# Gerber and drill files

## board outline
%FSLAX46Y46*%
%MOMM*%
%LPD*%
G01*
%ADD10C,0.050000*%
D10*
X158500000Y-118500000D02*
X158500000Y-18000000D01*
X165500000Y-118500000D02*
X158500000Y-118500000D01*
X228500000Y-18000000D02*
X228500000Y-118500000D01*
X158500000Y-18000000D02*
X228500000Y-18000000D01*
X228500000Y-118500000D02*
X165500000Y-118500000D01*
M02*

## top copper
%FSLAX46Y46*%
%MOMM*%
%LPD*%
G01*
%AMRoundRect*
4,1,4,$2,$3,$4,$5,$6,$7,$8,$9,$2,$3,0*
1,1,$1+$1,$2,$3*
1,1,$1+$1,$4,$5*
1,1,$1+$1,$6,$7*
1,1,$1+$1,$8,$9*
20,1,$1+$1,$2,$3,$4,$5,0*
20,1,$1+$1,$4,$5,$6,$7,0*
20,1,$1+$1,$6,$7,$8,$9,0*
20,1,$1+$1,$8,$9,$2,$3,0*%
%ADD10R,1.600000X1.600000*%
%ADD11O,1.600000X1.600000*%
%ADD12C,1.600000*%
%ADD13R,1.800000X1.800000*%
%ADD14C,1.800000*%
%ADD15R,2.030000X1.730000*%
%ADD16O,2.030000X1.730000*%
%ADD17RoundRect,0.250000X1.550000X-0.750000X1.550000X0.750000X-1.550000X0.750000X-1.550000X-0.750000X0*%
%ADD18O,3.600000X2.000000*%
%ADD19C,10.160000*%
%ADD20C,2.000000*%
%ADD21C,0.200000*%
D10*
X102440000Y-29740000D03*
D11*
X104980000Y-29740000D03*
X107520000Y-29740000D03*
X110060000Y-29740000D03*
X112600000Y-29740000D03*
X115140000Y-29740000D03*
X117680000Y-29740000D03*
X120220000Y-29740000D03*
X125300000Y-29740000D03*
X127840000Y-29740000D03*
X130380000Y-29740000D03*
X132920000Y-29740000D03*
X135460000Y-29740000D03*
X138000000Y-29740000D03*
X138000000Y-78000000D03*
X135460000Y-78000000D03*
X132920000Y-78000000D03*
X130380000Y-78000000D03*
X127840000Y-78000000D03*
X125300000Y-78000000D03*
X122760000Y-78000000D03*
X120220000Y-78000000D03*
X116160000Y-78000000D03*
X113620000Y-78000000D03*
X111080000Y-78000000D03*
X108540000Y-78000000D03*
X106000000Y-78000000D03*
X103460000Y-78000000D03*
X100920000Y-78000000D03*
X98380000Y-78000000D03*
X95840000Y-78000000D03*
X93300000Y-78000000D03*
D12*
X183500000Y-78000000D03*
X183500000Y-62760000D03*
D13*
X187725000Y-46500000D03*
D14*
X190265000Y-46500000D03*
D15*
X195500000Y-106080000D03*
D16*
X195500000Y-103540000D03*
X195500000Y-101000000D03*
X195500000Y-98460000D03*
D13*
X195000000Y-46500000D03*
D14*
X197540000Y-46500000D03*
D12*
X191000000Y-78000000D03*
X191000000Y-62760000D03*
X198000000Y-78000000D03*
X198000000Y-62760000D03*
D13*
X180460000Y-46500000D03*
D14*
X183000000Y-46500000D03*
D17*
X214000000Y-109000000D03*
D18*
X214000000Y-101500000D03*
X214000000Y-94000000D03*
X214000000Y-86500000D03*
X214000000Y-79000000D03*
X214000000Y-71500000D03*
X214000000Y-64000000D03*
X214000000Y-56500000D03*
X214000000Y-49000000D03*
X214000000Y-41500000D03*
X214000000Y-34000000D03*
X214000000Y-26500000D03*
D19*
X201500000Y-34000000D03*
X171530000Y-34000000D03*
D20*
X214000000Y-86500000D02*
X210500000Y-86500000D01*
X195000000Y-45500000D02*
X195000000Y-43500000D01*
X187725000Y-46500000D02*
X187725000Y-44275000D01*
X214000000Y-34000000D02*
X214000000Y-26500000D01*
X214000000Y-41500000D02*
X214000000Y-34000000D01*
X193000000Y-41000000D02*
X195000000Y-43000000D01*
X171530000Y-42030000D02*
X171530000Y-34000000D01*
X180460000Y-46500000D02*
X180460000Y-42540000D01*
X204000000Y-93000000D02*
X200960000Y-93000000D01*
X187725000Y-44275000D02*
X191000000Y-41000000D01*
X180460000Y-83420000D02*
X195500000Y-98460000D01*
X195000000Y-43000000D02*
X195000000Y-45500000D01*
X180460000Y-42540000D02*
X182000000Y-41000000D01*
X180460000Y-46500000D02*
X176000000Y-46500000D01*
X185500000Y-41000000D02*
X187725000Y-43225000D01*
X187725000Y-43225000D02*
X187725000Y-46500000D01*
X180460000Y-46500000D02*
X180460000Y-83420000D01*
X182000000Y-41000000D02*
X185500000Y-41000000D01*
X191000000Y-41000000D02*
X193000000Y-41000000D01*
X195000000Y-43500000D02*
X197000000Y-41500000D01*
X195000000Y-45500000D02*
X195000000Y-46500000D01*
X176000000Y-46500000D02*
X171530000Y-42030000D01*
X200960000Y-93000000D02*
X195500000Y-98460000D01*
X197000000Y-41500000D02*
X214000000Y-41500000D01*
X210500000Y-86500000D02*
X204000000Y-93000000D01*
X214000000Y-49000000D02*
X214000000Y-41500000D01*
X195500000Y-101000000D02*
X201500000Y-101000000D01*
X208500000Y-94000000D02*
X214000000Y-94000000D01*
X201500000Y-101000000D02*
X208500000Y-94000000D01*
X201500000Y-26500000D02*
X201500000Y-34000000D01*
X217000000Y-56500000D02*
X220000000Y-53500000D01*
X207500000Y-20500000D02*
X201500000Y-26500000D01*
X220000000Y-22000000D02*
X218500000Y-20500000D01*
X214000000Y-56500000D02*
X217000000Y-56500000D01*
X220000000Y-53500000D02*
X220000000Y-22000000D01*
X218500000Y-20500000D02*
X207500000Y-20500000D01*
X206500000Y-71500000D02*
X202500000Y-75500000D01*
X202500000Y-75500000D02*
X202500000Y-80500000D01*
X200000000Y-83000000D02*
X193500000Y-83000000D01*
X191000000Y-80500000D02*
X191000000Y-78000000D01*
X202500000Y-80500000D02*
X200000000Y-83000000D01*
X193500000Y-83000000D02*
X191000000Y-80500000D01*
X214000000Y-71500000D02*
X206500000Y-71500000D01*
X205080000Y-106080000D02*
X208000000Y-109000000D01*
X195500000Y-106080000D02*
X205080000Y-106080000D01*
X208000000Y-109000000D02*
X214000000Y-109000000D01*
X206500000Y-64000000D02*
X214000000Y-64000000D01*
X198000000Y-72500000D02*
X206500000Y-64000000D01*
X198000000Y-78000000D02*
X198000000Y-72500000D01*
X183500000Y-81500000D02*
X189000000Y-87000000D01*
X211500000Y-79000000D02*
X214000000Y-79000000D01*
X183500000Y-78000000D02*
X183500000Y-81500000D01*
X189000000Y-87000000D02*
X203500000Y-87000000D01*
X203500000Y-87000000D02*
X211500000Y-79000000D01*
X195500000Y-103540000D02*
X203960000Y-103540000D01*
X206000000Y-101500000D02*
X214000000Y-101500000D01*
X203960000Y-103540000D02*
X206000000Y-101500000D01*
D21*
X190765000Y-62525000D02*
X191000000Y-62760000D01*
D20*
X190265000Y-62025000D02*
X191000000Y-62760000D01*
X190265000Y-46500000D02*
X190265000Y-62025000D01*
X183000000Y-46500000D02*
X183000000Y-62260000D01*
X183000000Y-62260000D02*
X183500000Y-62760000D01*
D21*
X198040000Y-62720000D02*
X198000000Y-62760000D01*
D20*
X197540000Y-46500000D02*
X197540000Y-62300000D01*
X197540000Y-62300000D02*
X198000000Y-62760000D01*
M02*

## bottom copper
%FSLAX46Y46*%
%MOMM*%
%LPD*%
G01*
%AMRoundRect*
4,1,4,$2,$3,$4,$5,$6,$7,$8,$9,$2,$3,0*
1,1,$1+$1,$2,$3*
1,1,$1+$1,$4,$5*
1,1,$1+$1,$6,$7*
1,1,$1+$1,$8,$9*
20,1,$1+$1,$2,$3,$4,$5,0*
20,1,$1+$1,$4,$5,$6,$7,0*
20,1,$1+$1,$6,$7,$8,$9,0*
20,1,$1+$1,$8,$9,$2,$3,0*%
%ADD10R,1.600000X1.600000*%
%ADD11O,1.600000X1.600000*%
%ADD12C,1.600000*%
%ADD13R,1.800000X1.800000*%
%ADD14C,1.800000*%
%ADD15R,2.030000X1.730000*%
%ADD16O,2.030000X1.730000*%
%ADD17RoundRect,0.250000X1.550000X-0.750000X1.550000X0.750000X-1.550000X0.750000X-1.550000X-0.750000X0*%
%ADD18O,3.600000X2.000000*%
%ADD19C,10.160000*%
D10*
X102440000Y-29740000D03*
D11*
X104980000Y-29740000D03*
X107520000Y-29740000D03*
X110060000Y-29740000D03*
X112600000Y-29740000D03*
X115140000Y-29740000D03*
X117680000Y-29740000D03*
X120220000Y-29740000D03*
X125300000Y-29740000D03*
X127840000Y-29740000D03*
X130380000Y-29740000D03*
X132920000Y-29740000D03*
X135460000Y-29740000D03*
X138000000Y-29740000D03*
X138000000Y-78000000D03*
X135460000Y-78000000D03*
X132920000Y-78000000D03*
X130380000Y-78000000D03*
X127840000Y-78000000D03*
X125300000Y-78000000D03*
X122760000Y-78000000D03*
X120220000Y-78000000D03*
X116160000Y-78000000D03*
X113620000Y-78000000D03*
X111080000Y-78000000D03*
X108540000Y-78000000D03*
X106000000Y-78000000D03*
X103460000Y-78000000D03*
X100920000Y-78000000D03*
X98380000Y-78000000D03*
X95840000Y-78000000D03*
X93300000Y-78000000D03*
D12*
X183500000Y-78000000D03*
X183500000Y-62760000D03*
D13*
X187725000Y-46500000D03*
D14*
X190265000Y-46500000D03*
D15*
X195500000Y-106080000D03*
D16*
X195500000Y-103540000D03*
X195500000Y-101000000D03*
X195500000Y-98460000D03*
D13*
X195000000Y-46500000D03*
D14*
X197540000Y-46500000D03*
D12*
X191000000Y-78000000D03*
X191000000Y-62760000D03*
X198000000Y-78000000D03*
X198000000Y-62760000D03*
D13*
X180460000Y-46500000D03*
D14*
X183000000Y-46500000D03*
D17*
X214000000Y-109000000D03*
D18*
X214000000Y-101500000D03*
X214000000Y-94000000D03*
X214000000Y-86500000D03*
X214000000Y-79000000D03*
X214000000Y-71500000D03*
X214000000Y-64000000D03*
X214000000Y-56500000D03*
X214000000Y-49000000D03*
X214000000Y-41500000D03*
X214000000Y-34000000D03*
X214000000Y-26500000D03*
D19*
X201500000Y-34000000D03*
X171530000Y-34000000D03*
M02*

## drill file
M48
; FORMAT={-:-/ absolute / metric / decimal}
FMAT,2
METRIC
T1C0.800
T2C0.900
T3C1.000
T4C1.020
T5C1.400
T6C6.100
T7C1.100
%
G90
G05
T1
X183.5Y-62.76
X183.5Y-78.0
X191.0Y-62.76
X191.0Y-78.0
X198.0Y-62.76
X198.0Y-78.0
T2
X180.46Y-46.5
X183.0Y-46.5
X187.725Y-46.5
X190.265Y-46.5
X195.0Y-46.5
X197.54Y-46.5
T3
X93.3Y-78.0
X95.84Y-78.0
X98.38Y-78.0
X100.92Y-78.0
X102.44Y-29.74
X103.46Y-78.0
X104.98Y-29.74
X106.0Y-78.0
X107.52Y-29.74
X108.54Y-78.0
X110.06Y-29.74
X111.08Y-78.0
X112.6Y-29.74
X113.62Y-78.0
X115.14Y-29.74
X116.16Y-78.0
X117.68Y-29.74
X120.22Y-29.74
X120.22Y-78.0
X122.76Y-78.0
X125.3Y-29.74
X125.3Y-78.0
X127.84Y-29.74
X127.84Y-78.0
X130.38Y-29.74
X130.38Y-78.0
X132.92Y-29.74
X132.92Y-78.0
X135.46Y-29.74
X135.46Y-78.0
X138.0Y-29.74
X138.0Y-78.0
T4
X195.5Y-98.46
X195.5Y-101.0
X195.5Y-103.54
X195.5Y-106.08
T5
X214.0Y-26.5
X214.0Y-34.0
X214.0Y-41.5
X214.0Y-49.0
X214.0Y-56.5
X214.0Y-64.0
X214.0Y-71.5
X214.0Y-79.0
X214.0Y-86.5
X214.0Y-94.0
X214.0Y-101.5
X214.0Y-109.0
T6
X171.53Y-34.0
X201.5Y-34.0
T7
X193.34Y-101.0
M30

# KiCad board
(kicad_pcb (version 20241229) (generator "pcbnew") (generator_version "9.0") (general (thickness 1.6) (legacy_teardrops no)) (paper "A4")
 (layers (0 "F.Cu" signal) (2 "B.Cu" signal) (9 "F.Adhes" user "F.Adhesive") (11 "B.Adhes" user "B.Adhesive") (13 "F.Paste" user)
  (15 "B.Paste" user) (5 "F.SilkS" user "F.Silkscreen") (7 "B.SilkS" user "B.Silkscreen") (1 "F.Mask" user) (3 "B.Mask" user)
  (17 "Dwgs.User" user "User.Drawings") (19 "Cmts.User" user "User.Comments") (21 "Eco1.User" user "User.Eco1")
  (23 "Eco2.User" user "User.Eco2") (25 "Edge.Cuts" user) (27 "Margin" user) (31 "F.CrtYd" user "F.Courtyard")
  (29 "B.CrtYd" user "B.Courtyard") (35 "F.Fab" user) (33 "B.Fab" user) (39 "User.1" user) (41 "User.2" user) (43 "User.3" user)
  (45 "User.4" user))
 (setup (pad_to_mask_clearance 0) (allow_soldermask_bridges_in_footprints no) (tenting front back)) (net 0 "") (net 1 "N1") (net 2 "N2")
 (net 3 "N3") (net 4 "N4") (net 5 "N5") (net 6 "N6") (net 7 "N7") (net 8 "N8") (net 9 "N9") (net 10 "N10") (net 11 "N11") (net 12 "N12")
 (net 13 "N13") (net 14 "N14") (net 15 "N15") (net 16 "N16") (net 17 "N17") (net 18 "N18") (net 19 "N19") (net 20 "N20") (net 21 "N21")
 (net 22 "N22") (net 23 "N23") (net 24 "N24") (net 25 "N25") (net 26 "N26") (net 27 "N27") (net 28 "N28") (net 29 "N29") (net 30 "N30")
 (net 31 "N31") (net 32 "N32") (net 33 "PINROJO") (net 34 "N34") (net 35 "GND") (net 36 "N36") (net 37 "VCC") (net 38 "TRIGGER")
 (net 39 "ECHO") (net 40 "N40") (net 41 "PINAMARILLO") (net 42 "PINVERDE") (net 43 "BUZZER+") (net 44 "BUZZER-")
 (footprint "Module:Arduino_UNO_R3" (layer "F.Cu") (at 102.44 29.74)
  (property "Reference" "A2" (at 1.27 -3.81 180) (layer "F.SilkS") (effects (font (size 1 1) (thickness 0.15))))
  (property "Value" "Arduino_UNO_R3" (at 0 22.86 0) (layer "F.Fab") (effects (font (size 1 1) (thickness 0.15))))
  (pad "1" thru_hole rect (at 0 0 90) (size 1.6 1.6) (drill 1) (layers "*.Cu" "*.Mask") (remove_unused_layers no) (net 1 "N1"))
  (pad "2" thru_hole oval (at 2.54 0 90) (size 1.6 1.6) (drill 1) (layers "*.Cu" "*.Mask") (remove_unused_layers no) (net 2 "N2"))
  (pad "3" thru_hole oval (at 5.08 0 90) (size 1.6 1.6) (drill 1) (layers "*.Cu" "*.Mask") (remove_unused_layers no) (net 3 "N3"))
  (pad "4" thru_hole oval (at 7.62 0 90) (size 1.6 1.6) (drill 1) (layers "*.Cu" "*.Mask") (remove_unused_layers no) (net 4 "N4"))
  (pad "5" thru_hole oval (at 10.16 0 90) (size 1.6 1.6) (drill 1) (layers "*.Cu" "*.Mask") (remove_unused_layers no) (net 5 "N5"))
  (pad "6" thru_hole oval (at 12.7 0 90) (size 1.6 1.6) (drill 1) (layers "*.Cu" "*.Mask") (remove_unused_layers no) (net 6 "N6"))
  (pad "7" thru_hole oval (at 15.24 0 90) (size 1.6 1.6) (drill 1) (layers "*.Cu" "*.Mask") (remove_unused_layers no) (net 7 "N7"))
  (pad "8" thru_hole oval (at 17.78 0 90) (size 1.6 1.6) (drill 1) (layers "*.Cu" "*.Mask") (remove_unused_layers no) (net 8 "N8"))
  (pad "9" thru_hole oval (at 22.86 0 90) (size 1.6 1.6) (drill 1) (layers "*.Cu" "*.Mask") (remove_unused_layers no) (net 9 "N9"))
  (pad "10" thru_hole oval (at 25.4 0 90) (size 1.6 1.6) (drill 1) (layers "*.Cu" "*.Mask") (remove_unused_layers no) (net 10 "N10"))
  (pad "11" thru_hole oval (at 27.94 0 90) (size 1.6 1.6) (drill 1) (layers "*.Cu" "*.Mask") (remove_unused_layers no) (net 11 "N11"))
  (pad "12" thru_hole oval (at 30.48 0 90) (size 1.6 1.6) (drill 1) (layers "*.Cu" "*.Mask") (remove_unused_layers no) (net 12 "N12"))
  (pad "13" thru_hole oval (at 33.02 0 90) (size 1.6 1.6) (drill 1) (layers "*.Cu" "*.Mask") (remove_unused_layers no) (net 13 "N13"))
  (pad "14" thru_hole oval (at 35.56 0 90) (size 1.6 1.6) (drill 1) (layers "*.Cu" "*.Mask") (remove_unused_layers no) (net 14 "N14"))
  (pad "15" thru_hole oval (at 35.56 48.26 90) (size 1.6 1.6) (drill 1) (layers "*.Cu" "*.Mask") (remove_unused_layers no) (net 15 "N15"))
  (pad "16" thru_hole oval (at 33.02 48.26 90) (size 1.6 1.6) (drill 1) (layers "*.Cu" "*.Mask") (remove_unused_layers no) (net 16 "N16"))
  (pad "17" thru_hole oval (at 30.48 48.26 90) (size 1.6 1.6) (drill 1) (layers "*.Cu" "*.Mask") (remove_unused_layers no) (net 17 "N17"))
  (pad "18" thru_hole oval (at 27.94 48.26 90) (size 1.6 1.6) (drill 1) (layers "*.Cu" "*.Mask") (remove_unused_layers no) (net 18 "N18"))
  (pad "19" thru_hole oval (at 25.4 48.26 90) (size 1.6 1.6) (drill 1) (layers "*.Cu" "*.Mask") (remove_unused_layers no) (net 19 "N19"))
  (pad "20" thru_hole oval (at 22.86 48.26 90) (size 1.6 1.6) (drill 1) (layers "*.Cu" "*.Mask") (remove_unused_layers no) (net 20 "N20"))
  (pad "21" thru_hole oval (at 20.32 48.26 90) (size 1.6 1.6) (drill 1) (layers "*.Cu" "*.Mask") (remove_unused_layers no) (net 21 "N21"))
  (pad "22" thru_hole oval (at 17.78 48.26 90) (size 1.6 1.6) (drill 1) (layers "*.Cu" "*.Mask") (remove_unused_layers no) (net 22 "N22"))
  (pad "23" thru_hole oval (at 13.72 48.26 90) (size 1.6 1.6) (drill 1) (layers "*.Cu" "*.Mask") (remove_unused_layers no) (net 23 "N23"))
  (pad "24" thru_hole oval (at 11.18 48.26 90) (size 1.6 1.6) (drill 1) (layers "*.Cu" "*.Mask") (remove_unused_layers no) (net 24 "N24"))
  (pad "25" thru_hole oval (at 8.64 48.26 90) (size 1.6 1.6) (drill 1) (layers "*.Cu" "*.Mask") (remove_unused_layers no) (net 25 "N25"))
  (pad "26" thru_hole oval (at 6.1 48.26 90) (size 1.6 1.6) (drill 1) (layers "*.Cu" "*.Mask") (remove_unused_layers no) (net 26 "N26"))
  (pad "27" thru_hole oval (at 3.56 48.26 90) (size 1.6 1.6) (drill 1) (layers "*.Cu" "*.Mask") (remove_unused_layers no) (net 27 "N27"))
  (pad "28" thru_hole oval (at 1.02 48.26 90) (size 1.6 1.6) (drill 1) (layers "*.Cu" "*.Mask") (remove_unused_layers no) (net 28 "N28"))
  (pad "29" thru_hole oval (at -1.52 48.26 90) (size 1.6 1.6) (drill 1) (layers "*.Cu" "*.Mask") (remove_unused_layers no) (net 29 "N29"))
  (pad "30" thru_hole oval (at -4.06 48.26 90) (size 1.6 1.6) (drill 1) (layers "*.Cu" "*.Mask") (remove_unused_layers no) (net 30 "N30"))
  (pad "31" thru_hole oval (at -6.6 48.26 90) (size 1.6 1.6) (drill 1) (layers "*.Cu" "*.Mask") (remove_unused_layers no) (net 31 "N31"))
  (pad "32" thru_hole oval (at -9.14 48.26 90) (size 1.6 1.6) (drill 1) (layers "*.Cu" "*.Mask") (remove_unused_layers no) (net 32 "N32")))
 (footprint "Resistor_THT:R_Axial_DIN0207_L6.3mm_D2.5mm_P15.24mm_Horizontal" (layer "F.Cu") (at 183.5 78 90)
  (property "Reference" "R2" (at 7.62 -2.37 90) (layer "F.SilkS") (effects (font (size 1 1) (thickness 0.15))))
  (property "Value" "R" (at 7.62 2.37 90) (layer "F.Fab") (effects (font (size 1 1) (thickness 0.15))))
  (pad "1" thru_hole circle (at 0 0 90) (size 1.6 1.6) (drill 0.8) (layers "*.Cu" "*.Mask") (remove_unused_layers no) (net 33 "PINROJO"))
  (pad "2" thru_hole circle (at 15.24 0 90) (size 1.6 1.6) (drill 0.8) (layers "*.Cu" "*.Mask") (remove_unused_layers no) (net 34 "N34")))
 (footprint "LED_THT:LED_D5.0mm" (layer "F.Cu") (at 187.725 46.5)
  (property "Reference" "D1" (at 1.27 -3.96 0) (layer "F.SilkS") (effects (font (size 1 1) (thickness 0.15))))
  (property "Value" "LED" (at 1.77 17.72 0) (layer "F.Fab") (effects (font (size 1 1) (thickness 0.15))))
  (pad "1" thru_hole rect (at 0 0) (size 1.8 1.8) (drill 0.9) (layers "*.Cu" "*.Mask") (remove_unused_layers no) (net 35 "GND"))
  (pad "2" thru_hole circle (at 2.54 0) (size 1.8 1.8) (drill 0.9) (layers "*.Cu" "*.Mask") (remove_unused_layers no) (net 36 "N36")))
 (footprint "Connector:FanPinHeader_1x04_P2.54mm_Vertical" (layer "F.Cu") (at 195.5 106.08 90)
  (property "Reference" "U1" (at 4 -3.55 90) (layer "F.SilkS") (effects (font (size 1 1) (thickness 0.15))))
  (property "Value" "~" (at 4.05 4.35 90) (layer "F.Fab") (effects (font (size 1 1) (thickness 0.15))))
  (pad "" np_thru_hole circle (at 5.08 -2.16 180) (size 1.1 1.1) (drill 1.1) (layers "*.Cu" "*.Mask"))
  (pad "1" thru_hole rect (at 0 0 180) (size 2.03 1.73) (drill 1.02) (layers "*.Cu" "*.Mask") (remove_unused_layers no) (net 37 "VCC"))
  (pad "2" thru_hole oval (at 2.54 0 180) (size 2.03 1.73) (drill 1.02) (layers "*.Cu" "*.Mask") (remove_unused_layers no)
   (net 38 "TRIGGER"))
  (pad "3" thru_hole oval (at 5.08 0 180) (size 2.03 1.73) (drill 1.02) (layers "*.Cu" "*.Mask") (remove_unused_layers no) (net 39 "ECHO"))
  (pad "4" thru_hole oval (at 7.62 0 180) (size 2.03 1.73) (drill 1.02) (layers "*.Cu" "*.Mask") (remove_unused_layers no) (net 35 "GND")))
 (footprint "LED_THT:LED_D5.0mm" (layer "F.Cu") (at 195 46.5)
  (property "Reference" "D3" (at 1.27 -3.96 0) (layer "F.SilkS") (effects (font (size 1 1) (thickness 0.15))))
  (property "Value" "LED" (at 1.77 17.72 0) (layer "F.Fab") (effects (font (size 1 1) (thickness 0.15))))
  (pad "1" thru_hole rect (at 0 0) (size 1.8 1.8) (drill 0.9) (layers "*.Cu" "*.Mask") (remove_unused_layers no) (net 35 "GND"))
  (pad "2" thru_hole circle (at 2.54 0) (size 1.8 1.8) (drill 0.9) (layers "*.Cu" "*.Mask") (remove_unused_layers no) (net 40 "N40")))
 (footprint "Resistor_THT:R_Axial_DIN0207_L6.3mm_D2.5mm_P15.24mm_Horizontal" (layer "F.Cu") (at 191 78 90)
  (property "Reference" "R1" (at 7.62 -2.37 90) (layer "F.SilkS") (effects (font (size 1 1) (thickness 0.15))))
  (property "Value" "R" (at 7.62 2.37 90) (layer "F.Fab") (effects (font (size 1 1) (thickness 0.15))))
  (pad "1" thru_hole circle (at 0 0 90) (size 1.6 1.6) (drill 0.8) (layers "*.Cu" "*.Mask") (remove_unused_layers no) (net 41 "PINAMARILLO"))
  (pad "2" thru_hole circle (at 15.24 0 90) (size 1.6 1.6) (drill 0.8) (layers "*.Cu" "*.Mask") (remove_unused_layers no) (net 36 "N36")))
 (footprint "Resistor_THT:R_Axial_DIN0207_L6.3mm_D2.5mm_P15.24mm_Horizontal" (layer "F.Cu") (at 198 78 90)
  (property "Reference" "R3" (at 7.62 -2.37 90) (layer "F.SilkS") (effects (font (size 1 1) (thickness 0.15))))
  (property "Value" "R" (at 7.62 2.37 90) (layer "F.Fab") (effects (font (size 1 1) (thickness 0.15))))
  (pad "1" thru_hole circle (at 0 0 90) (size 1.6 1.6) (drill 0.8) (layers "*.Cu" "*.Mask") (remove_unused_layers no) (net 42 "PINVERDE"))
  (pad "2" thru_hole circle (at 15.24 0 90) (size 1.6 1.6) (drill 0.8) (layers "*.Cu" "*.Mask") (remove_unused_layers no) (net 40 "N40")))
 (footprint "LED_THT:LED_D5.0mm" (layer "F.Cu") (at 180.46 46.5)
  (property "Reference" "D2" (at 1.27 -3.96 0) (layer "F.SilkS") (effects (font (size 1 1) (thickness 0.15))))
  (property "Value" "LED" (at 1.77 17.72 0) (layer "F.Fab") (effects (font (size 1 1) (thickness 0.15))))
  (pad "1" thru_hole rect (at 0 0) (size 1.8 1.8) (drill 0.9) (layers "*.Cu" "*.Mask") (remove_unused_layers no) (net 35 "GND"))
  (pad "2" thru_hole circle (at 2.54 0) (size 1.8 1.8) (drill 0.9) (layers "*.Cu" "*.Mask") (remove_unused_layers no) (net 34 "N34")))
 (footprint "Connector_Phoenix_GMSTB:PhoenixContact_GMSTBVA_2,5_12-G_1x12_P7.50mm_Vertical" (layer "F.Cu") (at 214 109 90)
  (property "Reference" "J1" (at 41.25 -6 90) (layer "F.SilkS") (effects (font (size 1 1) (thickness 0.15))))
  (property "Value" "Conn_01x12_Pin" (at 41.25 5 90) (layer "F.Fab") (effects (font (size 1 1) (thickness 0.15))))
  (pad "1" thru_hole roundrect (at 0 0 90) (size 2 3.6) (drill 1.4) (layers "*.Cu" "*.Mask") (remove_unused_layers no)
   (roundrect_rratio 0.125) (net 37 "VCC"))
  (pad "2" thru_hole oval (at 7.5 0 90) (size 2 3.6) (drill 1.4) (layers "*.Cu" "*.Mask") (remove_unused_layers no) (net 38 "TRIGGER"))
  (pad "3" thru_hole oval (at 15 0 90) (size 2 3.6) (drill 1.4) (layers "*.Cu" "*.Mask") (remove_unused_layers no) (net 39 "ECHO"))
  (pad "4" thru_hole oval (at 22.5 0 90) (size 2 3.6) (drill 1.4) (layers "*.Cu" "*.Mask") (remove_unused_layers no) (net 35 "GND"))
  (pad "5" thru_hole oval (at 30 0 90) (size 2 3.6) (drill 1.4) (layers "*.Cu" "*.Mask") (remove_unused_layers no) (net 33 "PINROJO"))
  (pad "6" thru_hole oval (at 37.5 0 90) (size 2 3.6) (drill 1.4) (layers "*.Cu" "*.Mask") (remove_unused_layers no) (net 41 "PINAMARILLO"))
  (pad "7" thru_hole oval (at 45 0 90) (size 2 3.6) (drill 1.4) (layers "*.Cu" "*.Mask") (remove_unused_layers no) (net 42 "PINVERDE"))
  (pad "8" thru_hole oval (at 52.5 0 90) (size 2 3.6) (drill 1.4) (layers "*.Cu" "*.Mask") (remove_unused_layers no) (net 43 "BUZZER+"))
  (pad "9" thru_hole oval (at 60 0 90) (size 2 3.6) (drill 1.4) (layers "*.Cu" "*.Mask") (remove_unused_layers no) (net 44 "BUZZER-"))
  (pad "10" thru_hole oval (at 67.5 0 90) (size 2 3.6) (drill 1.4) (layers "*.Cu" "*.Mask") (remove_unused_layers no) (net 35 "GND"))
  (pad "11" thru_hole oval (at 75 0 90) (size 2 3.6) (drill 1.4) (layers "*.Cu" "*.Mask") (remove_unused_layers no) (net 35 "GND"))
  (pad "12" thru_hole oval (at 82.5 0 90) (size 2 3.6) (drill 1.4) (layers "*.Cu" "*.Mask") (remove_unused_layers no) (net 35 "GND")))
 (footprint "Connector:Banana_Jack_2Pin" (layer "F.Cu") (at 201.5 34 180)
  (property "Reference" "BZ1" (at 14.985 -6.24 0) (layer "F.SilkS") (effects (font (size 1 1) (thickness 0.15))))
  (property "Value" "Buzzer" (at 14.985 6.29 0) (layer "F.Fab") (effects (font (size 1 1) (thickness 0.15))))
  (pad "1" thru_hole circle (at 0 0 180) (size 10.16 10.16) (drill 6.1) (layers "*.Cu" "*.Mask") (remove_unused_layers no)
   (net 43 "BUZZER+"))
  (pad "2" thru_hole circle (at 29.97 0 180) (size 10.16 10.16) (drill 6.1) (layers "*.Cu" "*.Mask") (remove_unused_layers no)
   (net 44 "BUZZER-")))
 (gr_line (start 158.5 118.5) (end 158.5 18) (stroke (width 0.05) (type default)) (layer "Edge.Cuts"))
 (gr_line (start 165.5 118.5) (end 158.5 118.5) (stroke (width 0.05) (type default)) (layer "Edge.Cuts"))
 (gr_line (start 228.5 18) (end 228.5 118.5) (stroke (width 0.05) (type default)) (layer "Edge.Cuts"))
 (gr_line (start 158.5 18) (end 228.5 18) (stroke (width 0.05) (type default)) (layer "Edge.Cuts"))
 (gr_line (start 228.5 118.5) (end 165.5 118.5) (stroke (width 0.05) (type default)) (layer "Edge.Cuts"))
 (segment (start 214 86.5) (end 210.5 86.5) (width 2) (layer "F.Cu") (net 35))
 (segment (start 195 45.5) (end 195 43.5) (width 2) (layer "F.Cu") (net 35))
 (segment (start 187.725 46.5) (end 187.725 44.275) (width 2) (layer "F.Cu") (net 35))
 (segment (start 214 34) (end 214 26.5) (width 2) (layer "F.Cu") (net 35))
 (segment (start 214 41.5) (end 214 34) (width 2) (layer "F.Cu") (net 35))
 (segment (start 193 41) (end 195 43) (width 2) (layer "F.Cu") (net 35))
 (segment (start 171.53 42.03) (end 171.53 34) (width 2) (layer "F.Cu") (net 35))
 (segment (start 180.46 46.5) (end 180.46 42.54) (width 2) (layer "F.Cu") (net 35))
 (segment (start 204 93) (end 200.96 93) (width 2) (layer "F.Cu") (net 35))
 (segment (start 187.725 44.275) (end 191 41) (width 2) (layer "F.Cu") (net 35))
 (segment (start 180.46 83.42) (end 195.5 98.46) (width 2) (layer "F.Cu") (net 35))
 (segment (start 195 43) (end 195 45.5) (width 2) (layer "F.Cu") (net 35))
 (segment (start 180.46 42.54) (end 182 41) (width 2) (layer "F.Cu") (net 35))
 (segment (start 180.46 46.5) (end 176 46.5) (width 2) (layer "F.Cu") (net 35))
 (segment (start 185.5 41) (end 187.725 43.225) (width 2) (layer "F.Cu") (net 35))
 (segment (start 187.725 43.225) (end 187.725 46.5) (width 2) (layer "F.Cu") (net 35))
 (segment (start 180.46 46.5) (end 180.46 83.42) (width 2) (layer "F.Cu") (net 35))
 (segment (start 182 41) (end 185.5 41) (width 2) (layer "F.Cu") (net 35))
 (segment (start 191 41) (end 193 41) (width 2) (layer "F.Cu") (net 35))
 (segment (start 195 43.5) (end 197 41.5) (width 2) (layer "F.Cu") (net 35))
 (segment (start 195 45.5) (end 195 46.5) (width 2) (layer "F.Cu") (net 35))
 (segment (start 176 46.5) (end 171.53 42.03) (width 2) (layer "F.Cu") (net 35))
 (segment (start 200.96 93) (end 195.5 98.46) (width 2) (layer "F.Cu") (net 35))
 (segment (start 197 41.5) (end 214 41.5) (width 2) (layer "F.Cu") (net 35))
 (segment (start 210.5 86.5) (end 204 93) (width 2) (layer "F.Cu") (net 35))
 (segment (start 214 49) (end 214 41.5) (width 2) (layer "F.Cu") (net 35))
 (segment (start 195.5 101) (end 201.5 101) (width 2) (layer "F.Cu") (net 39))
 (segment (start 208.5 94) (end 214 94) (width 2) (layer "F.Cu") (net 39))
 (segment (start 201.5 101) (end 208.5 94) (width 2) (layer "F.Cu") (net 39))
 (segment (start 201.5 26.5) (end 201.5 34) (width 2) (layer "F.Cu") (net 43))
 (segment (start 217 56.5) (end 220 53.5) (width 2) (layer "F.Cu") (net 43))
 (segment (start 207.5 20.5) (end 201.5 26.5) (width 2) (layer "F.Cu") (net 43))
 (segment (start 220 22) (end 218.5 20.5) (width 2) (layer "F.Cu") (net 43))
 (segment (start 214 56.5) (end 217 56.5) (width 2) (layer "F.Cu") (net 43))
 (segment (start 220 53.5) (end 220 22) (width 2) (layer "F.Cu") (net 43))
 (segment (start 218.5 20.5) (end 207.5 20.5) (width 2) (layer "F.Cu") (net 43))
 (segment (start 206.5 71.5) (end 202.5 75.5) (width 2) (layer "F.Cu") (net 41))
 (segment (start 202.5 75.5) (end 202.5 80.5) (width 2) (layer "F.Cu") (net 41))
 (segment (start 200 83) (end 193.5 83) (width 2) (layer "F.Cu") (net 41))
 (segment (start 191 80.5) (end 191 78) (width 2) (layer "F.Cu") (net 41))
 (segment (start 202.5 80.5) (end 200 83) (width 2) (layer "F.Cu") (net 41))
 (segment (start 193.5 83) (end 191 80.5) (width 2) (layer "F.Cu") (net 41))
 (segment (start 214 71.5) (end 206.5 71.5) (width 2) (layer "F.Cu") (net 41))
 (segment (start 205.08 106.08) (end 208 109) (width 2) (layer "F.Cu") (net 37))
 (segment (start 195.5 106.08) (end 205.08 106.08) (width 2) (layer "F.Cu") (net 37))
 (segment (start 208 109) (end 214 109) (width 2) (layer "F.Cu") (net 37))
 (segment (start 206.5 64) (end 214 64) (width 2) (layer "F.Cu") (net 42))
 (segment (start 198 72.5) (end 206.5 64) (width 2) (layer "F.Cu") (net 42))
 (segment (start 198 78) (end 198 72.5) (width 2) (layer "F.Cu") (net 42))
 (segment (start 183.5 81.5) (end 189 87) (width 2) (layer "F.Cu") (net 33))
 (segment (start 211.5 79) (end 214 79) (width 2) (layer "F.Cu") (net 33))
 (segment (start 183.5 78) (end 183.5 81.5) (width 2) (layer "F.Cu") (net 33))
 (segment (start 189 87) (end 203.5 87) (width 2) (layer "F.Cu") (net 33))
 (segment (start 203.5 87) (end 211.5 79) (width 2) (layer "F.Cu") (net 33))
 (segment (start 195.5 103.54) (end 203.96 103.54) (width 2) (layer "F.Cu") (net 38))
 (segment (start 206 101.5) (end 214 101.5) (width 2) (layer "F.Cu") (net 38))
 (segment (start 203.96 103.54) (end 206 101.5) (width 2) (layer "F.Cu") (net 38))
 (segment (start 190.765 62.525) (end 191 62.76) (width 0.2) (layer "F.Cu") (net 36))
 (segment (start 190.265 62.025) (end 191 62.76) (width 2) (layer "F.Cu") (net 36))
 (segment (start 190.265 46.5) (end 190.265 62.025) (width 2) (layer "F.Cu") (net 36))
 (segment (start 183 46.5) (end 183 62.26) (width 2) (layer "F.Cu") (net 34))
 (segment (start 183 62.26) (end 183.5 62.76) (width 2) (layer "F.Cu") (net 34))
 (segment (start 198.04 62.72) (end 198 62.76) (width 0.2) (layer "F.Cu") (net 40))
 (segment (start 197.54 46.5) (end 197.54 62.3) (width 2) (layer "F.Cu") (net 40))
 (segment (start 197.54 62.3) (end 198 62.76) (width 2) (layer "F.Cu") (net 40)))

